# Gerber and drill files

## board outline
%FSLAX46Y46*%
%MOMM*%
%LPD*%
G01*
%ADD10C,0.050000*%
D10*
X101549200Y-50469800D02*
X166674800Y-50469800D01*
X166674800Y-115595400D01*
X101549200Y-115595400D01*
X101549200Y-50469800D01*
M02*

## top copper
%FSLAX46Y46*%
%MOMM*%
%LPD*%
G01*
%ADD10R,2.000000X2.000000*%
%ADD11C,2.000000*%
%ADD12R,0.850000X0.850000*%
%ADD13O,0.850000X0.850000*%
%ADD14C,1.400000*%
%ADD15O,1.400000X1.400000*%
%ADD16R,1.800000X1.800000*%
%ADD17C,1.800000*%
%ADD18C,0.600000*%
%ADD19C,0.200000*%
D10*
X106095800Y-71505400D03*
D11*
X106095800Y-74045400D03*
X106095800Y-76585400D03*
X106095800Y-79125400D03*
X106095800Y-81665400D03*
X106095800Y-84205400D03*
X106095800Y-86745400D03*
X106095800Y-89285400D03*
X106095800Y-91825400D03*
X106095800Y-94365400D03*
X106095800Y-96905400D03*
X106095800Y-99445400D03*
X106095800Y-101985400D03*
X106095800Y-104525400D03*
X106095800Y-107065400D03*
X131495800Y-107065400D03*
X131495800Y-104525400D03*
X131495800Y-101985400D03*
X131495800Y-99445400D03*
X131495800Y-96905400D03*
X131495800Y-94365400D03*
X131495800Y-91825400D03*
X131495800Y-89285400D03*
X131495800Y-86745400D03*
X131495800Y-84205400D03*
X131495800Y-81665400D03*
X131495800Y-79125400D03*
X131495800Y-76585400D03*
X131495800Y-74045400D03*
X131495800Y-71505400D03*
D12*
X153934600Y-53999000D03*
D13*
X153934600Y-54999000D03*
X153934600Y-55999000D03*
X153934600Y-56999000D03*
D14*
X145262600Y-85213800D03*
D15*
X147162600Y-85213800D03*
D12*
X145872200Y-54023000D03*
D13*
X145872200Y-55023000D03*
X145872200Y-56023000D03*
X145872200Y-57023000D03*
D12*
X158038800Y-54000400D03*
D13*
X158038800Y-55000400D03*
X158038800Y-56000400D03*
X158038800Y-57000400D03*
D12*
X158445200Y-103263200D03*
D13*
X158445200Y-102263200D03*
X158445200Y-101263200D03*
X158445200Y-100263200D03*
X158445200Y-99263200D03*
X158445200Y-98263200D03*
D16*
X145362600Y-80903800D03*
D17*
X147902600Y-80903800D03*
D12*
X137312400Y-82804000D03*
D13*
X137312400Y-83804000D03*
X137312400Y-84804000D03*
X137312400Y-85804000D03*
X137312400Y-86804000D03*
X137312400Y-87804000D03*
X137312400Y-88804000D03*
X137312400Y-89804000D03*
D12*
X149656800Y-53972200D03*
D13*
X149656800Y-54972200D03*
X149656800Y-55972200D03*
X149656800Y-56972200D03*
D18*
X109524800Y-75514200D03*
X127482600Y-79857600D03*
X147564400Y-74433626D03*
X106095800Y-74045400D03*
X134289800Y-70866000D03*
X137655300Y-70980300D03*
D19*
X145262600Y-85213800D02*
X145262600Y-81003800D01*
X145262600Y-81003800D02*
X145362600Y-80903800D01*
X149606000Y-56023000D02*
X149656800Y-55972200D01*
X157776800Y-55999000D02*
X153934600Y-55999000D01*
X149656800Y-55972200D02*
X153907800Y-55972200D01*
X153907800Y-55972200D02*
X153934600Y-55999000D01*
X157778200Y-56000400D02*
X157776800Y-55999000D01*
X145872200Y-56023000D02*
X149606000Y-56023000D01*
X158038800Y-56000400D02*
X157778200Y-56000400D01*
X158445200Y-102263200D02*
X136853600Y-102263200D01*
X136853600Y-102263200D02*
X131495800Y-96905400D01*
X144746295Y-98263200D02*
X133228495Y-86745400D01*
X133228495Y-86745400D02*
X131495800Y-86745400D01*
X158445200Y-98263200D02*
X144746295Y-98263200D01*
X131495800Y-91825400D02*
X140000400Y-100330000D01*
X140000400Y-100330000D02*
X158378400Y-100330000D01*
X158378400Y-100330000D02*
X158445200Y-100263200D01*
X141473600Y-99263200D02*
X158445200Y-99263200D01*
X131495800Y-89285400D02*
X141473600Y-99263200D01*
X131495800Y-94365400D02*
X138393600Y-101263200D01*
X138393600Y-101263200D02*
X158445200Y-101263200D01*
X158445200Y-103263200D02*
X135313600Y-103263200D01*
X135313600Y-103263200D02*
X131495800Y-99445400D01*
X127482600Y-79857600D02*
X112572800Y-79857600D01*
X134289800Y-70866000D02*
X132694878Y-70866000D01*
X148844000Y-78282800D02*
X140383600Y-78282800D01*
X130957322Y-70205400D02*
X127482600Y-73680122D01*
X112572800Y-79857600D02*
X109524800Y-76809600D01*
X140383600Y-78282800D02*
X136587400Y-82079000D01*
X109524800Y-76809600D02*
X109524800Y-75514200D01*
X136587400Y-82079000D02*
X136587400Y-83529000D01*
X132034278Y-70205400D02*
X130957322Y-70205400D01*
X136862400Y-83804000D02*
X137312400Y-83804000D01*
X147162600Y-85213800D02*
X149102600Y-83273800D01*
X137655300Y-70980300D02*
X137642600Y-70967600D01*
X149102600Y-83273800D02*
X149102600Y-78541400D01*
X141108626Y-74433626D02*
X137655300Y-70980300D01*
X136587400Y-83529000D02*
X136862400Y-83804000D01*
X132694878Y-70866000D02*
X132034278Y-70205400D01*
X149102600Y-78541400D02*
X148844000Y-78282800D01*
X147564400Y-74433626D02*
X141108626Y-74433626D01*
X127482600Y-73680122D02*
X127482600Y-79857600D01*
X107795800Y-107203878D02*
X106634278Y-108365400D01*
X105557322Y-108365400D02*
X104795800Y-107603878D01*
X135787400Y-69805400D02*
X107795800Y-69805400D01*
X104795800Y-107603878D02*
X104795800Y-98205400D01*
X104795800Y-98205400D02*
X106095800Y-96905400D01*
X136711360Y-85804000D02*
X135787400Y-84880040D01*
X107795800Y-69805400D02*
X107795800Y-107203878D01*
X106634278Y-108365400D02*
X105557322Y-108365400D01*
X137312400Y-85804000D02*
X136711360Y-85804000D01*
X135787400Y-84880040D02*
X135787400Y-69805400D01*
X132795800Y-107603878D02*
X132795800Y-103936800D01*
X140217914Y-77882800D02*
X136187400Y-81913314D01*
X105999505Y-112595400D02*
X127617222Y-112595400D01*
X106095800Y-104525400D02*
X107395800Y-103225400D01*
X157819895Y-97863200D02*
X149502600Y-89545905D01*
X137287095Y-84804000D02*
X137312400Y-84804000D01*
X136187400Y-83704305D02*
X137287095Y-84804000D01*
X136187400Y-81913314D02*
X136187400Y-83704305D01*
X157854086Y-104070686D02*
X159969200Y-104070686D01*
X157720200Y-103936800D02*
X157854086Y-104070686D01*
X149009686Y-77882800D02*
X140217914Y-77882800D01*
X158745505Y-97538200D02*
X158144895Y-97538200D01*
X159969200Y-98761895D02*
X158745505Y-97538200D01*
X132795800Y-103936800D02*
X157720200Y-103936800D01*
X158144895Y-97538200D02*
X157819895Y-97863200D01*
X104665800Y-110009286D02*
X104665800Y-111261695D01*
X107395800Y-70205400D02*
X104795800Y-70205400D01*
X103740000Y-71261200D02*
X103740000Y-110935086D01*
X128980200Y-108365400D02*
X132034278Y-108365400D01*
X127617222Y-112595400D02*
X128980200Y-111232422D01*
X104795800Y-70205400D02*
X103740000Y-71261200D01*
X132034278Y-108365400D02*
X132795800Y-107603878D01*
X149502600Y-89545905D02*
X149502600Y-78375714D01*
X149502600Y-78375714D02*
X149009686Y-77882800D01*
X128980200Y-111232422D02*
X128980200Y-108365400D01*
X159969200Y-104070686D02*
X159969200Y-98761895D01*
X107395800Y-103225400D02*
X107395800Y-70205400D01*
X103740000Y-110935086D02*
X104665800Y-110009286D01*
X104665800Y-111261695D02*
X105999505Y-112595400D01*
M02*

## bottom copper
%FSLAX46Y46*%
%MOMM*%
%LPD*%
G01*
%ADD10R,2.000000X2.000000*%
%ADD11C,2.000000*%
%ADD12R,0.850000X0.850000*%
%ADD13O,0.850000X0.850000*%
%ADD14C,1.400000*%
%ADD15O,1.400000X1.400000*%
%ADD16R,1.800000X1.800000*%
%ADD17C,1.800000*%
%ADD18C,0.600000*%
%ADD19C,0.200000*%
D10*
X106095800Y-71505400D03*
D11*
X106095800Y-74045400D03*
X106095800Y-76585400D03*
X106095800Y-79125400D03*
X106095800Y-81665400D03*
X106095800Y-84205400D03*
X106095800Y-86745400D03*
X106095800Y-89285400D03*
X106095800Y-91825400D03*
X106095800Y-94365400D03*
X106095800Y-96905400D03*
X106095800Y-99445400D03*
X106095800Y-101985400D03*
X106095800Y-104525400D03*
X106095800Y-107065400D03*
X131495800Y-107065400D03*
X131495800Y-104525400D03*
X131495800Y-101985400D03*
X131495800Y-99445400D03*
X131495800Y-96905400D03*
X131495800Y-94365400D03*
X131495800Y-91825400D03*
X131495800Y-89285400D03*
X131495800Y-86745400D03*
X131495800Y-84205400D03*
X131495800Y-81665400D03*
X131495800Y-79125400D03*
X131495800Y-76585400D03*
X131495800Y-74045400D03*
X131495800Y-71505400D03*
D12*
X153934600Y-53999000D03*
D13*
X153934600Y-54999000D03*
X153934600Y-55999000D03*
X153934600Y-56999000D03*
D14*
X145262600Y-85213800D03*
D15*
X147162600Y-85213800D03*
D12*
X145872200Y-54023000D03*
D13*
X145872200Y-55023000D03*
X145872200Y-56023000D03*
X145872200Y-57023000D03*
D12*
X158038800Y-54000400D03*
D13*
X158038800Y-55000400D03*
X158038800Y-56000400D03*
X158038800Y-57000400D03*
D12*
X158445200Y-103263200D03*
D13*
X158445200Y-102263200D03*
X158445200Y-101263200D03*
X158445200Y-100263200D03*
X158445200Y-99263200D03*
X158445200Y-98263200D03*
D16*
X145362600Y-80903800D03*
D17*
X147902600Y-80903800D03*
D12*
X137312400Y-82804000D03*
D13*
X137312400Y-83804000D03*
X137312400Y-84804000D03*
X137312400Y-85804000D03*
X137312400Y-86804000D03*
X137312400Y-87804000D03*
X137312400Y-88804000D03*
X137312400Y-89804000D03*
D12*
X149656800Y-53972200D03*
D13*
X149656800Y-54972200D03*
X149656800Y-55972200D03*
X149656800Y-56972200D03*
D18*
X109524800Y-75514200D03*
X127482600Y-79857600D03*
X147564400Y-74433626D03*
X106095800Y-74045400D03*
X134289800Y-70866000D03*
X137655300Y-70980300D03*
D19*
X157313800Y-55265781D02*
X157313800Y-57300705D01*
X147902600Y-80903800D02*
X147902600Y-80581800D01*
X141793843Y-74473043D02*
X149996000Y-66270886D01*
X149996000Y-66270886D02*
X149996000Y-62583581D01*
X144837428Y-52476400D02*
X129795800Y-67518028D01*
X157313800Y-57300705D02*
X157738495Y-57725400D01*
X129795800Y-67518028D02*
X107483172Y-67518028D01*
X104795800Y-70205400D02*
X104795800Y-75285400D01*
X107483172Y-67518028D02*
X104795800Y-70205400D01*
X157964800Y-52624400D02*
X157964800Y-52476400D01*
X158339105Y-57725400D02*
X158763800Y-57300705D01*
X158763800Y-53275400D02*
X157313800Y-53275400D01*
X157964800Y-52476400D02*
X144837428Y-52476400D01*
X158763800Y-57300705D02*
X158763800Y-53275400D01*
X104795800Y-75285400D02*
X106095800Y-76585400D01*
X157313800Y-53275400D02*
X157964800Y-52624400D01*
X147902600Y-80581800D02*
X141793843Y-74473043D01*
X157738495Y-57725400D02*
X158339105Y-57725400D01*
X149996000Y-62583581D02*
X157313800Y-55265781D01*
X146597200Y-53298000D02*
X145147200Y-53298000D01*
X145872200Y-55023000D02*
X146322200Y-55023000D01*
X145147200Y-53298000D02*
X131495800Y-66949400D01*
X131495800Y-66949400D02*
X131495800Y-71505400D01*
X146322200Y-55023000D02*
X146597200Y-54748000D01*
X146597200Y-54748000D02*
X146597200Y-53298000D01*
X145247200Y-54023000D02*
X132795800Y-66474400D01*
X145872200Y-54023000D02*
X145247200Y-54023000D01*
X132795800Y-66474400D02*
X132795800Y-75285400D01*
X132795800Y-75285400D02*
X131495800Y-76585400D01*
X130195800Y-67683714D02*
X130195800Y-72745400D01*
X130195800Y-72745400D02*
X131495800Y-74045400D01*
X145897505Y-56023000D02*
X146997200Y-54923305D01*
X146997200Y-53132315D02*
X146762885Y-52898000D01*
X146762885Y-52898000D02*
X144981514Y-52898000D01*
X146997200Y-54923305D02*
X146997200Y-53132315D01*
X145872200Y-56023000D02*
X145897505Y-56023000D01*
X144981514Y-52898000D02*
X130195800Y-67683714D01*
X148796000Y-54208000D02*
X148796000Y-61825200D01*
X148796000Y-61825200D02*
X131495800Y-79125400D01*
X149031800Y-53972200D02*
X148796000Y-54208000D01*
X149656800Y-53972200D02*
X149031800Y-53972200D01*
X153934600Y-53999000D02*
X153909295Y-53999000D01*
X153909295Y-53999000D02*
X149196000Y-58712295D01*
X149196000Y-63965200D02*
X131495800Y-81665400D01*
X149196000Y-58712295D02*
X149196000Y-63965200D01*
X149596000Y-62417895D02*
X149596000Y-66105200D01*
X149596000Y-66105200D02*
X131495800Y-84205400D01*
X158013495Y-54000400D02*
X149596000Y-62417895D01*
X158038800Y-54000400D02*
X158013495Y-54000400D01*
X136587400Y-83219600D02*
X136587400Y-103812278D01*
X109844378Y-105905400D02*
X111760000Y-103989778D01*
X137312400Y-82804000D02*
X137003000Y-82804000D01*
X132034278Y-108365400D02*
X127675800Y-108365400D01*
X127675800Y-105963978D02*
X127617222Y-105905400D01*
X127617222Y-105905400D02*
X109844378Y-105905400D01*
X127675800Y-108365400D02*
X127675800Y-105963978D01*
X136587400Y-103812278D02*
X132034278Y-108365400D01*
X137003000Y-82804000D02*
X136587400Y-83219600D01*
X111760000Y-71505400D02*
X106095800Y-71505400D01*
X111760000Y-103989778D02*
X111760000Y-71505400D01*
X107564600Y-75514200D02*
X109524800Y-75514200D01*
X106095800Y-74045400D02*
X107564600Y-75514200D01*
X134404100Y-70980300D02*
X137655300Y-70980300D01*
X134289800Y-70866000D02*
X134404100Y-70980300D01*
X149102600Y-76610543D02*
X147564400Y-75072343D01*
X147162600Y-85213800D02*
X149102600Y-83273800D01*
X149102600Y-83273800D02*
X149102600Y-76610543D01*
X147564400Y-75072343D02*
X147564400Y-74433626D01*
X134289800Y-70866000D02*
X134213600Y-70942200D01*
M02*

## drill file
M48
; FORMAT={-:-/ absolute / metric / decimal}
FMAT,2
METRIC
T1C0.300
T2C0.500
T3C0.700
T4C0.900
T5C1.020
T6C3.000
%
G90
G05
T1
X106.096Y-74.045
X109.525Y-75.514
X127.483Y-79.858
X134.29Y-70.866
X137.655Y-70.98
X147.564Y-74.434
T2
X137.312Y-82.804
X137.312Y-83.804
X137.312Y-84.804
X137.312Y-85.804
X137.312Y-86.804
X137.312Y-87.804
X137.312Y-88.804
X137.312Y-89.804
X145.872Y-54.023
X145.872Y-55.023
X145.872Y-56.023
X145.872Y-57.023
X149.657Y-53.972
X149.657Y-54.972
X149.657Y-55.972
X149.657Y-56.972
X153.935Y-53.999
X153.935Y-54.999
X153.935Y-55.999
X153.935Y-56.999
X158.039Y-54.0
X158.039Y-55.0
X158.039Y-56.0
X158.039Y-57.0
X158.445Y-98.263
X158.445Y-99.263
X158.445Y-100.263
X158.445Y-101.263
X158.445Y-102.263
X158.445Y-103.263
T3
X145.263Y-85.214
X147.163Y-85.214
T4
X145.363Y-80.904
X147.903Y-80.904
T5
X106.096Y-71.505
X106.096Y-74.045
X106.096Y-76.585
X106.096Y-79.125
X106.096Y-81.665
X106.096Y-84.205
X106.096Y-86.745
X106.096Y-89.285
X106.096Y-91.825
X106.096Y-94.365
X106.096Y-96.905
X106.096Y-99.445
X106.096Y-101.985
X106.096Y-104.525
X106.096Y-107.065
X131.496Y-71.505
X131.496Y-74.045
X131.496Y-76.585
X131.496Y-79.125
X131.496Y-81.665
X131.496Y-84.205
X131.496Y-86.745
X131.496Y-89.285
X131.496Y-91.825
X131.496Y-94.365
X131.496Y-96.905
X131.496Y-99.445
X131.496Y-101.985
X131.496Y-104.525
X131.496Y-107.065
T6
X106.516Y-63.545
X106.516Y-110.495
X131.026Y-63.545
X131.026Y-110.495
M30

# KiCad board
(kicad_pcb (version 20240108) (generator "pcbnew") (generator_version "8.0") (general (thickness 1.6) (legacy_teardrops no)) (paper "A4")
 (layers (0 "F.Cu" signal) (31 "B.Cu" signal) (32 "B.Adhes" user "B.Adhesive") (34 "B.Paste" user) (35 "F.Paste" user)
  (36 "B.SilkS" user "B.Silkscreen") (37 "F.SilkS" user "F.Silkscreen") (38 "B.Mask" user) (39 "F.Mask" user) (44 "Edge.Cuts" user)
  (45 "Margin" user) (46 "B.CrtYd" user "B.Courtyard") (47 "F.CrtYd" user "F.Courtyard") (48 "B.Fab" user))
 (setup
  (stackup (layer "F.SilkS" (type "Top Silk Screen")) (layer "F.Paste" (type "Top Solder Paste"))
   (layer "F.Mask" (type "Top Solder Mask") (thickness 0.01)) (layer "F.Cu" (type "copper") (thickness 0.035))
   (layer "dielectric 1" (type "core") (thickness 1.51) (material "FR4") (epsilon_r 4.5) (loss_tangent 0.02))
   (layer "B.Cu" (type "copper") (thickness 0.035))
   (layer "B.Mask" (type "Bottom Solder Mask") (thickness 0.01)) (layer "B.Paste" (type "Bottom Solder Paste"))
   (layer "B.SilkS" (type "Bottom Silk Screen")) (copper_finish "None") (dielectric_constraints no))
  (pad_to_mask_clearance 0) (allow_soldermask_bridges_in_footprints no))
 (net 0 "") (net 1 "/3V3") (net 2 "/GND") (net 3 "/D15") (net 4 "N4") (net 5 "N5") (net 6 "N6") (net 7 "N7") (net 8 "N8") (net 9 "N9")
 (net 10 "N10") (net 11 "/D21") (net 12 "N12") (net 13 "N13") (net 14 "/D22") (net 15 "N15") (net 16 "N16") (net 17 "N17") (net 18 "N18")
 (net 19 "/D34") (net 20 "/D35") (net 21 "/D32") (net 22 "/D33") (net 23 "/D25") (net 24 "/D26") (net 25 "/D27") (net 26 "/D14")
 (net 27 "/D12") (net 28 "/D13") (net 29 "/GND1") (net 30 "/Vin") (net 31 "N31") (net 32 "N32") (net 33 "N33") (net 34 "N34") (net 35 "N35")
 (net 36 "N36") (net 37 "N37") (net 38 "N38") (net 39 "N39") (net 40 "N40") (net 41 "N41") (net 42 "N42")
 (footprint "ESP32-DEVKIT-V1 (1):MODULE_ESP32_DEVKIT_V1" (layer "F.Cu") (at 118.7958 87.0204)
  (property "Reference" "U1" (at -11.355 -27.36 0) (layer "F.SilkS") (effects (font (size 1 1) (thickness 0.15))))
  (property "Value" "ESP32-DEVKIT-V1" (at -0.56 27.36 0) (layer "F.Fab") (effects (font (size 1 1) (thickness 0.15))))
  (pad "" np_thru_hole circle (at -12.28 -23.475) (size 3 3) (drill 3) (layers "*.Cu" "*.Mask"))
  (pad "" np_thru_hole circle (at -12.28 23.475) (size 3 3) (drill 3) (layers "*.Cu" "*.Mask"))
  (pad "" np_thru_hole circle (at 12.23 -23.475) (size 3 3) (drill 3) (layers "*.Cu" "*.Mask"))
  (pad "" np_thru_hole circle (at 12.23 23.475) (size 3 3) (drill 3) (layers "*.Cu" "*.Mask"))
  (pad "1" thru_hole rect (at -12.7 -15.515) (size 2 2) (drill 1.02) (layers "*.Cu" "*.Mask") (remove_unused_layers no) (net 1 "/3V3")
   (solder_mask_margin 0.102))
  (pad "2" thru_hole circle (at -12.7 -12.975) (size 2 2) (drill 1.02) (layers "*.Cu" "*.Mask") (remove_unused_layers no) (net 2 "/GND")
   (solder_mask_margin 0.102))
  (pad "3" thru_hole circle (at -12.7 -10.435) (size 2 2) (drill 1.02) (layers "*.Cu" "*.Mask") (remove_unused_layers no) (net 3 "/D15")
   (solder_mask_margin 0.102))
  (pad "4" thru_hole circle (at -12.7 -7.895) (size 2 2) (drill 1.02) (layers "*.Cu" "*.Mask") (remove_unused_layers no) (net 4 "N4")
   (solder_mask_margin 0.102))
  (pad "5" thru_hole circle (at -12.7 -5.355) (size 2 2) (drill 1.02) (layers "*.Cu" "*.Mask") (remove_unused_layers no) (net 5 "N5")
   (solder_mask_margin 0.102))
  (pad "6" thru_hole circle (at -12.7 -2.815) (size 2 2) (drill 1.02) (layers "*.Cu" "*.Mask") (remove_unused_layers no) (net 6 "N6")
   (solder_mask_margin 0.102))
  (pad "7" thru_hole circle (at -12.7 -0.275) (size 2 2) (drill 1.02) (layers "*.Cu" "*.Mask") (remove_unused_layers no) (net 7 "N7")
   (solder_mask_margin 0.102))
  (pad "8" thru_hole circle (at -12.7 2.265) (size 2 2) (drill 1.02) (layers "*.Cu" "*.Mask") (remove_unused_layers no) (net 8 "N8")
   (solder_mask_margin 0.102))
  (pad "9" thru_hole circle (at -12.7 4.805) (size 2 2) (drill 1.02) (layers "*.Cu" "*.Mask") (remove_unused_layers no) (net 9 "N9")
   (solder_mask_margin 0.102))
  (pad "10" thru_hole circle (at -12.7 7.345) (size 2 2) (drill 1.02) (layers "*.Cu" "*.Mask") (remove_unused_layers no) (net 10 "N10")
   (solder_mask_margin 0.102))
  (pad "11" thru_hole circle (at -12.7 9.885) (size 2 2) (drill 1.02) (layers "*.Cu" "*.Mask") (remove_unused_layers no) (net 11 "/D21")
   (solder_mask_margin 0.102))
  (pad "12" thru_hole circle (at -12.7 12.425) (size 2 2) (drill 1.02) (layers "*.Cu" "*.Mask") (remove_unused_layers no) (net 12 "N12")
   (solder_mask_margin 0.102))
  (pad "13" thru_hole circle (at -12.7 14.965) (size 2 2) (drill 1.02) (layers "*.Cu" "*.Mask") (remove_unused_layers no) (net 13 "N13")
   (solder_mask_margin 0.102))
  (pad "14" thru_hole circle (at -12.7 17.505) (size 2 2) (drill 1.02) (layers "*.Cu" "*.Mask") (remove_unused_layers no) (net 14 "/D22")
   (solder_mask_margin 0.102))
  (pad "15" thru_hole circle (at -12.7 20.045) (size 2 2) (drill 1.02) (layers "*.Cu" "*.Mask") (remove_unused_layers no) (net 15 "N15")
   (solder_mask_margin 0.102))
  (pad "16" thru_hole circle (at 12.7 20.045) (size 2 2) (drill 1.02) (layers "*.Cu" "*.Mask") (remove_unused_layers no) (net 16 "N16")
   (solder_mask_margin 0.102))
  (pad "17" thru_hole circle (at 12.7 17.505) (size 2 2) (drill 1.02) (layers "*.Cu" "*.Mask") (remove_unused_layers no) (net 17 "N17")
   (solder_mask_margin 0.102))
  (pad "18" thru_hole circle (at 12.7 14.965) (size 2 2) (drill 1.02) (layers "*.Cu" "*.Mask") (remove_unused_layers no) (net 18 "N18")
   (solder_mask_margin 0.102))
  (pad "19" thru_hole circle (at 12.7 12.425) (size 2 2) (drill 1.02) (layers "*.Cu" "*.Mask") (remove_unused_layers no) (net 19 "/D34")
   (solder_mask_margin 0.102))
  (pad "20" thru_hole circle (at 12.7 9.885) (size 2 2) (drill 1.02) (layers "*.Cu" "*.Mask") (remove_unused_layers no) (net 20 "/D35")
   (solder_mask_margin 0.102))
  (pad "21" thru_hole circle (at 12.7 7.345) (size 2 2) (drill 1.02) (layers "*.Cu" "*.Mask") (remove_unused_layers no) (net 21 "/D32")
   (solder_mask_margin 0.102))
  (pad "22" thru_hole circle (at 12.7 4.805) (size 2 2) (drill 1.02) (layers "*.Cu" "*.Mask") (remove_unused_layers no) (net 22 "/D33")
   (solder_mask_margin 0.102))
  (pad "23" thru_hole circle (at 12.7 2.265) (size 2 2) (drill 1.02) (layers "*.Cu" "*.Mask") (remove_unused_layers no) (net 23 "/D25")
   (solder_mask_margin 0.102))
  (pad "24" thru_hole circle (at 12.7 -0.275) (size 2 2) (drill 1.02) (layers "*.Cu" "*.Mask") (remove_unused_layers no) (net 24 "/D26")
   (solder_mask_margin 0.102))
  (pad "25" thru_hole circle (at 12.7 -2.815) (size 2 2) (drill 1.02) (layers "*.Cu" "*.Mask") (remove_unused_layers no) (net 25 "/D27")
   (solder_mask_margin 0.102))
  (pad "26" thru_hole circle (at 12.7 -5.355) (size 2 2) (drill 1.02) (layers "*.Cu" "*.Mask") (remove_unused_layers no) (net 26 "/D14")
   (solder_mask_margin 0.102))
  (pad "27" thru_hole circle (at 12.7 -7.895) (size 2 2) (drill 1.02) (layers "*.Cu" "*.Mask") (remove_unused_layers no) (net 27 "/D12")
   (solder_mask_margin 0.102))
  (pad "28" thru_hole circle (at 12.7 -10.435) (size 2 2) (drill 1.02) (layers "*.Cu" "*.Mask") (remove_unused_layers no) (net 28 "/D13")
   (solder_mask_margin 0.102))
  (pad "29" thru_hole circle (at 12.7 -12.975) (size 2 2) (drill 1.02) (layers "*.Cu" "*.Mask") (remove_unused_layers no) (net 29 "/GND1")
   (solder_mask_margin 0.102))
  (pad "30" thru_hole circle (at 12.7 -15.515) (size 2 2) (drill 1.02) (layers "*.Cu" "*.Mask") (remove_unused_layers no) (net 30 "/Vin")
   (solder_mask_margin 0.102))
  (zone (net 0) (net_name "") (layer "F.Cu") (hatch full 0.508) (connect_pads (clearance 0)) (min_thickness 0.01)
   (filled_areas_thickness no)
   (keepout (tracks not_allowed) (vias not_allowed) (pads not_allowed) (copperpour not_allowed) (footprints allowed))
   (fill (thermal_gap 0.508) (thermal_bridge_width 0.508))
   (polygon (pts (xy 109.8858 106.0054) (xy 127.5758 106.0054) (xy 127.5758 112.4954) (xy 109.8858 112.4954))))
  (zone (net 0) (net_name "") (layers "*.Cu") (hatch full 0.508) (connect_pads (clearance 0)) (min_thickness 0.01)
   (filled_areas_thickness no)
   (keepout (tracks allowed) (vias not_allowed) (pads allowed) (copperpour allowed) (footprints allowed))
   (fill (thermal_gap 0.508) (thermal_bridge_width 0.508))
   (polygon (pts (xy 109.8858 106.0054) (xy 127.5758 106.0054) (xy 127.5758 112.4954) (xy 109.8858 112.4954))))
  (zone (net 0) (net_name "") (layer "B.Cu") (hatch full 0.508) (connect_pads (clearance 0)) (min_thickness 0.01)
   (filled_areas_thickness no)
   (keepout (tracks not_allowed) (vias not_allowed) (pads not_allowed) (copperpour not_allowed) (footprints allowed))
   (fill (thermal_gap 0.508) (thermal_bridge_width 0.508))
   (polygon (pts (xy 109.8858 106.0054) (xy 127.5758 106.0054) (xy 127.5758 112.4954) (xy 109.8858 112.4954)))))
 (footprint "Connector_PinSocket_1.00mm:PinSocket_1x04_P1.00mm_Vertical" (layer "F.Cu") (at 153.9346 53.999)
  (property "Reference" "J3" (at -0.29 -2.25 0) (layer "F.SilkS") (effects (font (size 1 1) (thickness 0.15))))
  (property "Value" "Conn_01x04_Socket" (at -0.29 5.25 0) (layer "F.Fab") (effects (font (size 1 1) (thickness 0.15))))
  (pad "1" thru_hole rect (at 0 0) (size 0.85 0.85) (drill 0.5) (layers "*.Cu" "*.Mask") (remove_unused_layers no) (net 26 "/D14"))
  (pad "2" thru_hole oval (at 0 1) (size 0.85 0.85) (drill 0.5) (layers "*.Cu" "*.Mask") (remove_unused_layers no) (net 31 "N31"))
  (pad "3" thru_hole oval (at 0 2) (size 0.85 0.85) (drill 0.5) (layers "*.Cu" "*.Mask") (remove_unused_layers no) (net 29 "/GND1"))
  (pad "4" thru_hole oval (at 0 3) (size 0.85 0.85) (drill 0.5) (layers "*.Cu" "*.Mask") (remove_unused_layers no) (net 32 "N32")))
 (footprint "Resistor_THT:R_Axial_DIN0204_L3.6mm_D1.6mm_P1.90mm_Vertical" (layer "F.Cu") (at 145.2626 85.2138)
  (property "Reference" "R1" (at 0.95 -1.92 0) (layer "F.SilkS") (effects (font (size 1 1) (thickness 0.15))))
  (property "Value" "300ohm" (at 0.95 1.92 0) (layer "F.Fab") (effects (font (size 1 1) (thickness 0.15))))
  (pad "1" thru_hole circle (at 0 0) (size 1.4 1.4) (drill 0.7) (layers "*.Cu" "*.Mask") (remove_unused_layers no) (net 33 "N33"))
  (pad "2" thru_hole oval (at 1.9 0) (size 1.4 1.4) (drill 0.7) (layers "*.Cu" "*.Mask") (remove_unused_layers no) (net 2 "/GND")))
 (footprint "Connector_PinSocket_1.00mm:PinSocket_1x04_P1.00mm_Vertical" (layer "F.Cu") (at 145.8722 54.023)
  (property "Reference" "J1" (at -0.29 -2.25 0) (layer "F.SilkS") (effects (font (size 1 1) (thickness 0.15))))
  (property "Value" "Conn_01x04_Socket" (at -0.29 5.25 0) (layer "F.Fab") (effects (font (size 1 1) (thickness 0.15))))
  (pad "1" thru_hole rect (at 0 0) (size 0.85 0.85) (drill 0.5) (layers "*.Cu" "*.Mask") (remove_unused_layers no) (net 28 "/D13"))
  (pad "2" thru_hole oval (at 0 1) (size 0.85 0.85) (drill 0.5) (layers "*.Cu" "*.Mask") (remove_unused_layers no) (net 30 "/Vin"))
  (pad "3" thru_hole oval (at 0 2) (size 0.85 0.85) (drill 0.5) (layers "*.Cu" "*.Mask") (remove_unused_layers no) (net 29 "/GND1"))
  (pad "4" thru_hole oval (at 0 3) (size 0.85 0.85) (drill 0.5) (layers "*.Cu" "*.Mask") (remove_unused_layers no) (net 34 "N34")))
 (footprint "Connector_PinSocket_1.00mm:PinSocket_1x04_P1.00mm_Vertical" (layer "F.Cu") (at 158.0388 54.0004)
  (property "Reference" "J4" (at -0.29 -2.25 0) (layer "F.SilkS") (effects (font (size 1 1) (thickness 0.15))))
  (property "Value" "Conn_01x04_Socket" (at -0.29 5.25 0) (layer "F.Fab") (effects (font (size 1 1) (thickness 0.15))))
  (pad "1" thru_hole rect (at 0 0) (size 0.85 0.85) (drill 0.5) (layers "*.Cu" "*.Mask") (remove_unused_layers no) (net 25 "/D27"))
  (pad "2" thru_hole oval (at 0 1) (size 0.85 0.85) (drill 0.5) (layers "*.Cu" "*.Mask") (remove_unused_layers no) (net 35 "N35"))
  (pad "3" thru_hole oval (at 0 2) (size 0.85 0.85) (drill 0.5) (layers "*.Cu" "*.Mask") (remove_unused_layers no) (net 29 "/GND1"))
  (pad "4" thru_hole oval (at 0 3) (size 0.85 0.85) (drill 0.5) (layers "*.Cu" "*.Mask") (remove_unused_layers no) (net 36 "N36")))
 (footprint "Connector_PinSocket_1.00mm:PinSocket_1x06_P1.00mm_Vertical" (layer "F.Cu") (at 158.4452 103.2632 180)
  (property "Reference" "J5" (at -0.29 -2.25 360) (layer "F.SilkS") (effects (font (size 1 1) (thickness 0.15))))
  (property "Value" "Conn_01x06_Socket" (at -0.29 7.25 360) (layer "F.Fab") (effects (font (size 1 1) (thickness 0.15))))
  (pad "1" thru_hole rect (at 0 0 180) (size 0.85 0.85) (drill 0.5) (layers "*.Cu" "*.Mask") (remove_unused_layers no) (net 19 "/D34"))
  (pad "2" thru_hole oval (at 0 1 180) (size 0.85 0.85) (drill 0.5) (layers "*.Cu" "*.Mask") (remove_unused_layers no) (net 20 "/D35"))
  (pad "3" thru_hole oval (at 0 2 180) (size 0.85 0.85) (drill 0.5) (layers "*.Cu" "*.Mask") (remove_unused_layers no) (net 21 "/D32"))
  (pad "4" thru_hole oval (at 0 3 180) (size 0.85 0.85) (drill 0.5) (layers "*.Cu" "*.Mask") (remove_unused_layers no) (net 22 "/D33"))
  (pad "5" thru_hole oval (at 0 4 180) (size 0.85 0.85) (drill 0.5) (layers "*.Cu" "*.Mask") (remove_unused_layers no) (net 23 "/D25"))
  (pad "6" thru_hole oval (at 0 5 180) (size 0.85 0.85) (drill 0.5) (layers "*.Cu" "*.Mask") (remove_unused_layers no) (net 24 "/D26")))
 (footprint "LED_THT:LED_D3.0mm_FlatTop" (layer "F.Cu") (at 145.3626 80.9038)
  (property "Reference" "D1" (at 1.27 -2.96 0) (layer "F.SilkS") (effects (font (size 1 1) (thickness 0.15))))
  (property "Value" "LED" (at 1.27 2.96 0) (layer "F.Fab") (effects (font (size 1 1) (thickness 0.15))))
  (pad "1" thru_hole rect (at 0 0) (size 1.8 1.8) (drill 0.9) (layers "*.Cu" "*.Mask") (remove_unused_layers no) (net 33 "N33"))
  (pad "2" thru_hole circle (at 2.54 0) (size 1.8 1.8) (drill 0.9) (layers "*.Cu" "*.Mask") (remove_unused_layers no) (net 3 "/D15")))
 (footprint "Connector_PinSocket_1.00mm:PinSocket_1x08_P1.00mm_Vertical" (layer "F.Cu") (at 137.3124 82.804)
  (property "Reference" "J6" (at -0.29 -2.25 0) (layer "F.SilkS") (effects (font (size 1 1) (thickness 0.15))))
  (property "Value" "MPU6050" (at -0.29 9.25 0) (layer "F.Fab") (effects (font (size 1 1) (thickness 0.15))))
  (pad "1" thru_hole rect (at 0 0) (size 0.85 0.85) (drill 0.5) (layers "*.Cu" "*.Mask") (remove_unused_layers no) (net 1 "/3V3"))
  (pad "2" thru_hole oval (at 0 1) (size 0.85 0.85) (drill 0.5) (layers "*.Cu" "*.Mask") (remove_unused_layers no) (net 2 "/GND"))
  (pad "3" thru_hole oval (at 0 2) (size 0.85 0.85) (drill 0.5) (layers "*.Cu" "*.Mask") (remove_unused_layers no) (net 14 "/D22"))
  (pad "4" thru_hole oval (at 0 3) (size 0.85 0.85) (drill 0.5) (layers "*.Cu" "*.Mask") (remove_unused_layers no) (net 11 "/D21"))
  (pad "5" thru_hole oval (at 0 4) (size 0.85 0.85) (drill 0.5) (layers "*.Cu" "*.Mask") (remove_unused_layers no) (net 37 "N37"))
  (pad "6" thru_hole oval (at 0 5) (size 0.85 0.85) (drill 0.5) (layers "*.Cu" "*.Mask") (remove_unused_layers no) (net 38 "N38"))
  (pad "7" thru_hole oval (at 0 6) (size 0.85 0.85) (drill 0.5) (layers "*.Cu" "*.Mask") (remove_unused_layers no) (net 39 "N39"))
  (pad "8" thru_hole oval (at 0 7) (size 0.85 0.85) (drill 0.5) (layers "*.Cu" "*.Mask") (remove_unused_layers no) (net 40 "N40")))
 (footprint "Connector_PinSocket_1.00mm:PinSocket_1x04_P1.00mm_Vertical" (layer "F.Cu") (at 149.6568 53.9722)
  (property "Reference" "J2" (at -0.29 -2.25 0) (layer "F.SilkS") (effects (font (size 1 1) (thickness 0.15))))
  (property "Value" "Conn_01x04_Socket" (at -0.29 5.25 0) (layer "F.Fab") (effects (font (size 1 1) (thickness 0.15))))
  (pad "1" thru_hole rect (at 0 0) (size 0.85 0.85) (drill 0.5) (layers "*.Cu" "*.Mask") (remove_unused_layers no) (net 27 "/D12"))
  (pad "2" thru_hole oval (at 0 1) (size 0.85 0.85) (drill 0.5) (layers "*.Cu" "*.Mask") (remove_unused_layers no) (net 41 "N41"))
  (pad "3" thru_hole oval (at 0 2) (size 0.85 0.85) (drill 0.5) (layers "*.Cu" "*.Mask") (remove_unused_layers no) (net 29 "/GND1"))
  (pad "4" thru_hole oval (at 0 3) (size 0.85 0.85) (drill 0.5) (layers "*.Cu" "*.Mask") (remove_unused_layers no) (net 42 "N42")))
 (gr_rect (start 101.5492 50.4698) (end 166.6748 115.5954) (stroke (width 0.05) (type default)) (fill none) (layer "Edge.Cuts"))
 (segment (start 145.2626 85.2138) (end 145.2626 81.0038) (width 0.2) (layer "F.Cu") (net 33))
 (segment (start 145.2626 81.0038) (end 145.3626 80.9038) (width 0.2) (layer "F.Cu") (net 33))
 (segment (start 157.3138 55.265781) (end 157.3138 57.300705) (width 0.2) (layer "B.Cu") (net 3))
 (segment (start 147.9026 80.9038) (end 147.9026 80.5818) (width 0.2) (layer "B.Cu") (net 3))
 (segment (start 141.793843 74.473043) (end 149.996 66.270886) (width 0.2) (layer "B.Cu") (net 3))
 (segment (start 149.996 66.270886) (end 149.996 62.583581) (width 0.2) (layer "B.Cu") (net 3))
 (segment (start 144.837428 52.4764) (end 129.7958 67.518028) (width 0.2) (layer "B.Cu") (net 3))
 (segment (start 157.3138 57.300705) (end 157.738495 57.7254) (width 0.2) (layer "B.Cu") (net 3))
 (segment (start 129.7958 67.518028) (end 107.483172 67.518028) (width 0.2) (layer "B.Cu") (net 3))
 (segment (start 104.7958 70.2054) (end 104.7958 75.2854) (width 0.2) (layer "B.Cu") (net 3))
 (segment (start 107.483172 67.518028) (end 104.7958 70.2054) (width 0.2) (layer "B.Cu") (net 3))
 (segment (start 157.9648 52.6244) (end 157.9648 52.4764) (width 0.2) (layer "B.Cu") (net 3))
 (segment (start 158.339105 57.7254) (end 158.7638 57.300705) (width 0.2) (layer "B.Cu") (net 3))
 (segment (start 158.7638 53.2754) (end 157.3138 53.2754) (width 0.2) (layer "B.Cu") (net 3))
 (segment (start 157.9648 52.4764) (end 144.837428 52.4764) (width 0.2) (layer "B.Cu") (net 3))
 (segment (start 158.7638 57.300705) (end 158.7638 53.2754) (width 0.2) (layer "B.Cu") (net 3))
 (segment (start 104.7958 75.2854) (end 106.0958 76.5854) (width 0.2) (layer "B.Cu") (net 3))
 (segment (start 157.3138 53.2754) (end 157.9648 52.6244) (width 0.2) (layer "B.Cu") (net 3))
 (segment (start 147.9026 80.5818) (end 141.793843 74.473043) (width 0.2) (layer "B.Cu") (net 3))
 (segment (start 157.738495 57.7254) (end 158.339105 57.7254) (width 0.2) (layer "B.Cu") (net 3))
 (segment (start 149.996 62.583581) (end 157.3138 55.265781) (width 0.2) (layer "B.Cu") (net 3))
 (segment (start 146.5972 53.298) (end 145.1472 53.298) (width 0.2) (layer "B.Cu") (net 30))
 (segment (start 145.8722 55.023) (end 146.3222 55.023) (width 0.2) (layer "B.Cu") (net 30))
 (segment (start 145.1472 53.298) (end 131.4958 66.9494) (width 0.2) (layer "B.Cu") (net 30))
 (segment (start 131.4958 66.9494) (end 131.4958 71.5054) (width 0.2) (layer "B.Cu") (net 30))
 (segment (start 146.3222 55.023) (end 146.5972 54.748) (width 0.2) (layer "B.Cu") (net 30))
 (segment (start 146.5972 54.748) (end 146.5972 53.298) (width 0.2) (layer "B.Cu") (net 30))
 (segment (start 145.2472 54.023) (end 132.7958 66.4744) (width 0.2) (layer "B.Cu") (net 28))
 (segment (start 145.8722 54.023) (end 145.2472 54.023) (width 0.2) (layer "B.Cu") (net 28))
 (segment (start 132.7958 66.4744) (end 132.7958 75.2854) (width 0.2) (layer "B.Cu") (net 28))
 (segment (start 132.7958 75.2854) (end 131.4958 76.5854) (width 0.2) (layer "B.Cu") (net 28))
 (segment (start 149.606 56.023) (end 149.6568 55.9722) (width 0.2) (layer "F.Cu") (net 29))
 (segment (start 157.7768 55.999) (end 153.9346 55.999) (width 0.2) (layer "F.Cu") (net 29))
 (segment (start 149.6568 55.9722) (end 153.9078 55.9722) (width 0.2) (layer "F.Cu") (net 29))
 (segment (start 153.9078 55.9722) (end 153.9346 55.999) (width 0.2) (layer "F.Cu") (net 29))
 (segment (start 157.7782 56.0004) (end 157.7768 55.999) (width 0.2) (layer "F.Cu") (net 29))
 (segment (start 145.8722 56.023) (end 149.606 56.023) (width 0.2) (layer "F.Cu") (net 29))
 (segment (start 158.0388 56.0004) (end 157.7782 56.0004) (width 0.2) (layer "F.Cu") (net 29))
 (segment (start 130.1958 67.683714) (end 130.1958 72.7454) (width 0.2) (layer "B.Cu") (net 29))
 (segment (start 130.1958 72.7454) (end 131.4958 74.0454) (width 0.2) (layer "B.Cu") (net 29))
 (segment (start 145.897505 56.023) (end 146.9972 54.923305) (width 0.2) (layer "B.Cu") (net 29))
 (segment (start 146.9972 53.132315) (end 146.762885 52.898) (width 0.2) (layer "B.Cu") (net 29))
 (segment (start 146.762885 52.898) (end 144.981514 52.898) (width 0.2) (layer "B.Cu") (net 29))
 (segment (start 146.9972 54.923305) (end 146.9972 53.132315) (width 0.2) (layer "B.Cu") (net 29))
 (segment (start 145.8722 56.023) (end 145.897505 56.023) (width 0.2) (layer "B.Cu") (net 29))
 (segment (start 144.981514 52.898) (end 130.1958 67.683714) (width 0.2) (layer "B.Cu") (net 29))
 (segment (start 148.796 54.208) (end 148.796 61.8252) (width 0.2) (layer "B.Cu") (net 27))
 (segment (start 148.796 61.8252) (end 131.4958 79.1254) (width 0.2) (layer "B.Cu") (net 27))
 (segment (start 149.0318 53.9722) (end 148.796 54.208) (width 0.2) (layer "B.Cu") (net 27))
 (segment (start 149.6568 53.9722) (end 149.0318 53.9722) (width 0.2) (layer "B.Cu") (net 27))
 (segment (start 153.9346 53.999) (end 153.909295 53.999) (width 0.2) (layer "B.Cu") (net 26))
 (segment (start 153.909295 53.999) (end 149.196 58.712295) (width 0.2) (layer "B.Cu") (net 26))
 (segment (start 149.196 63.9652) (end 131.4958 81.6654) (width 0.2) (layer "B.Cu") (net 26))
 (segment (start 149.196 58.712295) (end 149.196 63.9652) (width 0.2) (layer "B.Cu") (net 26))
 (segment (start 149.596 62.417895) (end 149.596 66.1052) (width 0.2) (layer "B.Cu") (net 25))
 (segment (start 149.596 66.1052) (end 131.4958 84.2054) (width 0.2) (layer "B.Cu") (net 25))
 (segment (start 158.013495 54.0004) (end 149.596 62.417895) (width 0.2) (layer "B.Cu") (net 25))
 (segment (start 158.0388 54.0004) (end 158.013495 54.0004) (width 0.2) (layer "B.Cu") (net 25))
 (segment (start 158.4452 102.2632) (end 136.8536 102.2632) (width 0.2) (layer "F.Cu") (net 20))
 (segment (start 136.8536 102.2632) (end 131.4958 96.9054) (width 0.2) (layer "F.Cu") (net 20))
 (segment (start 144.746295 98.2632) (end 133.228495 86.7454) (width 0.2) (layer "F.Cu") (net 24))
 (segment (start 133.228495 86.7454) (end 131.4958 86.7454) (width 0.2) (layer "F.Cu") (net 24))
 (segment (start 158.4452 98.2632) (end 144.746295 98.2632) (width 0.2) (layer "F.Cu") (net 24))
 (segment (start 131.4958 91.8254) (end 140.0004 100.33) (width 0.2) (layer "F.Cu") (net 22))
 (segment (start 140.0004 100.33) (end 158.3784 100.33) (width 0.2) (layer "F.Cu") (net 22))
 (segment (start 158.3784 100.33) (end 158.4452 100.2632) (width 0.2) (layer "F.Cu") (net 22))
 (segment (start 141.4736 99.2632) (end 158.4452 99.2632) (width 0.2) (layer "F.Cu") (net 23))
 (segment (start 131.4958 89.2854) (end 141.4736 99.2632) (width 0.2) (layer "F.Cu") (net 23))
 (segment (start 131.4958 94.3654) (end 138.3936 101.2632) (width 0.2) (layer "F.Cu") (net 21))
 (segment (start 138.3936 101.2632) (end 158.4452 101.2632) (width 0.2) (layer "F.Cu") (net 21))
 (segment (start 158.4452 103.2632) (end 135.3136 103.2632) (width 0.2) (layer "F.Cu") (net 19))
 (segment (start 135.3136 103.2632) (end 131.4958 99.4454) (width 0.2) (layer "F.Cu") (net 19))
 (segment (start 136.5874 83.2196) (end 136.5874 103.812278) (width 0.2) (layer "B.Cu") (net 1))
 (segment (start 109.844378 105.9054) (end 111.76 103.989778) (width 0.2) (layer "B.Cu") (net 1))
 (segment (start 137.3124 82.804) (end 137.003 82.804) (width 0.2) (layer "B.Cu") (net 1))
 (segment (start 132.034278 108.3654) (end 127.6758 108.3654) (width 0.2) (layer "B.Cu") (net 1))
 (segment (start 127.6758 105.963978) (end 127.617222 105.9054) (width 0.2) (layer "B.Cu") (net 1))
 (segment (start 127.617222 105.9054) (end 109.844378 105.9054) (width 0.2) (layer "B.Cu") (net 1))
 (segment (start 127.6758 108.3654) (end 127.6758 105.963978) (width 0.2) (layer "B.Cu") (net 1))
 (segment (start 136.5874 103.812278) (end 132.034278 108.3654) (width 0.2) (layer "B.Cu") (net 1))
 (segment (start 137.003 82.804) (end 136.5874 83.2196) (width 0.2) (layer "B.Cu") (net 1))
 (segment (start 111.76 71.5054) (end 106.0958 71.5054) (width 0.2) (layer "B.Cu") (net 1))
 (segment (start 111.76 103.989778) (end 111.76 71.5054) (width 0.2) (layer "B.Cu") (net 1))
 (segment (start 127.4826 79.8576) (end 112.5728 79.8576) (width 0.2) (layer "F.Cu") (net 2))
 (segment (start 134.2898 70.866) (end 132.694878 70.866) (width 0.2) (layer "F.Cu") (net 2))
 (segment (start 148.844 78.2828) (end 140.3836 78.2828) (width 0.2) (layer "F.Cu") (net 2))
 (segment (start 130.957322 70.2054) (end 127.4826 73.680122) (width 0.2) (layer "F.Cu") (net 2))
 (segment (start 112.5728 79.8576) (end 109.5248 76.8096) (width 0.2) (layer "F.Cu") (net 2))
 (segment (start 140.3836 78.2828) (end 136.5874 82.079) (width 0.2) (layer "F.Cu") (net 2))
 (segment (start 109.5248 76.8096) (end 109.5248 75.5142) (width 0.2) (layer "F.Cu") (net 2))
 (segment (start 136.5874 82.079) (end 136.5874 83.529) (width 0.2) (layer "F.Cu") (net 2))
 (segment (start 132.034278 70.2054) (end 130.957322 70.2054) (width 0.2) (layer "F.Cu") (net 2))
 (segment (start 136.8624 83.804) (end 137.3124 83.804) (width 0.2) (layer "F.Cu") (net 2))
 (segment (start 147.1626 85.2138) (end 149.1026 83.2738) (width 0.2) (layer "F.Cu") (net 2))
 (segment (start 137.6553 70.9803) (end 137.6426 70.9676) (width 0.2) (layer "F.Cu") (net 2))
 (segment (start 149.1026 83.2738) (end 149.1026 78.5414) (width 0.2) (layer "F.Cu") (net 2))
 (segment (start 141.108626 74.433626) (end 137.6553 70.9803) (width 0.2) (layer "F.Cu") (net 2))
 (segment (start 136.5874 83.529) (end 136.8624 83.804) (width 0.2) (layer "F.Cu") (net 2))
 (segment (start 132.694878 70.866) (end 132.034278 70.2054) (width 0.2) (layer "F.Cu") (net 2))
 (segment (start 149.1026 78.5414) (end 148.844 78.2828) (width 0.2) (layer "F.Cu") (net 2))
 (segment (start 147.5644 74.433626) (end 141.108626 74.433626) (width 0.2) (layer "F.Cu") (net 2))
 (segment (start 127.4826 73.680122) (end 127.4826 79.8576) (width 0.2) (layer "F.Cu") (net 2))
 (via (at 109.5248 75.5142) (size 0.6) (drill 0.3) (layers "F.Cu" "B.Cu") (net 2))
 (via (at 127.4826 79.8576) (size 0.6) (drill 0.3) (layers "F.Cu" "B.Cu") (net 2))
 (via (at 147.5644 74.433626) (size 0.6) (drill 0.3) (layers "F.Cu" "B.Cu") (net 2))
 (via (at 106.0958 74.0454) (size 0.6) (drill 0.3) (layers "F.Cu" "B.Cu") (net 2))
 (via (at 134.2898 70.866) (size 0.6) (drill 0.3) (layers "F.Cu" "B.Cu") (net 2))
 (via (at 137.6553 70.9803) (size 0.6) (drill 0.3) (layers "F.Cu" "B.Cu") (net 2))
 (segment (start 107.5646 75.5142) (end 109.5248 75.5142) (width 0.2) (layer "B.Cu") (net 2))
 (segment (start 106.0958 74.0454) (end 107.5646 75.5142) (width 0.2) (layer "B.Cu") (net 2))
 (segment (start 134.4041 70.9803) (end 137.6553 70.9803) (width 0.2) (layer "B.Cu") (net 2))
 (segment (start 134.2898 70.866) (end 134.4041 70.9803) (width 0.2) (layer "B.Cu") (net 2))
 (segment (start 149.1026 76.610543) (end 147.5644 75.072343) (width 0.2) (layer "B.Cu") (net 2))
 (segment (start 147.1626 85.2138) (end 149.1026 83.2738) (width 0.2) (layer "B.Cu") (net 2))
 (segment (start 149.1026 83.2738) (end 149.1026 76.610543) (width 0.2) (layer "B.Cu") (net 2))
 (segment (start 147.5644 75.072343) (end 147.5644 74.433626) (width 0.2) (layer "B.Cu") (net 2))
 (segment (start 134.2898 70.866) (end 134.2136 70.9422) (width 0.2) (layer "B.Cu") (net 2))
 (segment (start 107.7958 107.203878) (end 106.634278 108.3654) (width 0.2) (layer "F.Cu") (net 11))
 (segment (start 105.557322 108.3654) (end 104.7958 107.603878) (width 0.2) (layer "F.Cu") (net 11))
 (segment (start 135.7874 69.8054) (end 107.7958 69.8054) (width 0.2) (layer "F.Cu") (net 11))
 (segment (start 104.7958 107.603878) (end 104.7958 98.2054) (width 0.2) (layer "F.Cu") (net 11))
 (segment (start 104.7958 98.2054) (end 106.0958 96.9054) (width 0.2) (layer "F.Cu") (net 11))
 (segment (start 136.71136 85.804) (end 135.7874 84.88004) (width 0.2) (layer "F.Cu") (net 11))
 (segment (start 107.7958 69.8054) (end 107.7958 107.203878) (width 0.2) (layer "F.Cu") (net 11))
 (segment (start 106.634278 108.3654) (end 105.557322 108.3654) (width 0.2) (layer "F.Cu") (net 11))
 (segment (start 137.3124 85.804) (end 136.71136 85.804) (width 0.2) (layer "F.Cu") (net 11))
 (segment (start 135.7874 84.88004) (end 135.7874 69.8054) (width 0.2) (layer "F.Cu") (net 11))
 (segment (start 132.7958 107.603878) (end 132.7958 103.9368) (width 0.2) (layer "F.Cu") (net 14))
 (segment (start 140.217914 77.8828) (end 136.1874 81.913314) (width 0.2) (layer "F.Cu") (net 14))
 (segment (start 105.999505 112.5954) (end 127.617222 112.5954) (width 0.2) (layer "F.Cu") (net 14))
 (segment (start 106.0958 104.5254) (end 107.3958 103.2254) (width 0.2) (layer "F.Cu") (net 14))
 (segment (start 157.819895 97.8632) (end 149.5026 89.545905) (width 0.2) (layer "F.Cu") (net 14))
 (segment (start 137.287095 84.804) (end 137.3124 84.804) (width 0.2) (layer "F.Cu") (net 14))
 (segment (start 136.1874 83.704305) (end 137.287095 84.804) (width 0.2) (layer "F.Cu") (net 14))
 (segment (start 136.1874 81.913314) (end 136.1874 83.704305) (width 0.2) (layer "F.Cu") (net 14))
 (segment (start 157.854086 104.070686) (end 159.9692 104.070686) (width 0.2) (layer "F.Cu") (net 14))
 (segment (start 157.7202 103.9368) (end 157.854086 104.070686) (width 0.2) (layer "F.Cu") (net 14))
 (segment (start 149.009686 77.8828) (end 140.217914 77.8828) (width 0.2) (layer "F.Cu") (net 14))
 (segment (start 158.745505 97.5382) (end 158.144895 97.5382) (width 0.2) (layer "F.Cu") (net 14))
 (segment (start 159.9692 98.761895) (end 158.745505 97.5382) (width 0.2) (layer "F.Cu") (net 14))
 (segment (start 132.7958 103.9368) (end 157.7202 103.9368) (width 0.2) (layer "F.Cu") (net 14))
 (segment (start 158.144895 97.5382) (end 157.819895 97.8632) (width 0.2) (layer "F.Cu") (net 14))
 (segment (start 104.6658 110.009286) (end 104.6658 111.261695) (width 0.2) (layer "F.Cu") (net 14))
 (segment (start 107.3958 70.2054) (end 104.7958 70.2054) (width 0.2) (layer "F.Cu") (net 14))
 (segment (start 103.74 71.2612) (end 103.74 110.935086) (width 0.2) (layer "F.Cu") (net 14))
 (segment (start 128.9802 108.3654) (end 132.034278 108.3654) (width 0.2) (layer "F.Cu") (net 14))
 (segment (start 127.617222 112.5954) (end 128.9802 111.232422) (width 0.2) (layer "F.Cu") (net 14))
 (segment (start 104.7958 70.2054) (end 103.74 71.2612) (width 0.2) (layer "F.Cu") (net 14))
 (segment (start 132.034278 108.3654) (end 132.7958 107.603878) (width 0.2) (layer "F.Cu") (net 14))
 (segment (start 149.5026 89.545905) (end 149.5026 78.375714) (width 0.2) (layer "F.Cu") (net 14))
 (segment (start 149.5026 78.375714) (end 149.009686 77.8828) (width 0.2) (layer "F.Cu") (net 14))
 (segment (start 128.9802 111.232422) (end 128.9802 108.3654) (width 0.2) (layer "F.Cu") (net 14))
 (segment (start 159.9692 104.070686) (end 159.9692 98.761895) (width 0.2) (layer "F.Cu") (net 14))
 (segment (start 107.3958 103.2254) (end 107.3958 70.2054) (width 0.2) (layer "F.Cu") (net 14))
 (segment (start 103.74 110.935086) (end 104.6658 110.009286) (width 0.2) (layer "F.Cu") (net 14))
 (segment (start 104.6658 111.261695) (end 105.999505 112.5954) (width 0.2) (layer "F.Cu") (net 14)))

